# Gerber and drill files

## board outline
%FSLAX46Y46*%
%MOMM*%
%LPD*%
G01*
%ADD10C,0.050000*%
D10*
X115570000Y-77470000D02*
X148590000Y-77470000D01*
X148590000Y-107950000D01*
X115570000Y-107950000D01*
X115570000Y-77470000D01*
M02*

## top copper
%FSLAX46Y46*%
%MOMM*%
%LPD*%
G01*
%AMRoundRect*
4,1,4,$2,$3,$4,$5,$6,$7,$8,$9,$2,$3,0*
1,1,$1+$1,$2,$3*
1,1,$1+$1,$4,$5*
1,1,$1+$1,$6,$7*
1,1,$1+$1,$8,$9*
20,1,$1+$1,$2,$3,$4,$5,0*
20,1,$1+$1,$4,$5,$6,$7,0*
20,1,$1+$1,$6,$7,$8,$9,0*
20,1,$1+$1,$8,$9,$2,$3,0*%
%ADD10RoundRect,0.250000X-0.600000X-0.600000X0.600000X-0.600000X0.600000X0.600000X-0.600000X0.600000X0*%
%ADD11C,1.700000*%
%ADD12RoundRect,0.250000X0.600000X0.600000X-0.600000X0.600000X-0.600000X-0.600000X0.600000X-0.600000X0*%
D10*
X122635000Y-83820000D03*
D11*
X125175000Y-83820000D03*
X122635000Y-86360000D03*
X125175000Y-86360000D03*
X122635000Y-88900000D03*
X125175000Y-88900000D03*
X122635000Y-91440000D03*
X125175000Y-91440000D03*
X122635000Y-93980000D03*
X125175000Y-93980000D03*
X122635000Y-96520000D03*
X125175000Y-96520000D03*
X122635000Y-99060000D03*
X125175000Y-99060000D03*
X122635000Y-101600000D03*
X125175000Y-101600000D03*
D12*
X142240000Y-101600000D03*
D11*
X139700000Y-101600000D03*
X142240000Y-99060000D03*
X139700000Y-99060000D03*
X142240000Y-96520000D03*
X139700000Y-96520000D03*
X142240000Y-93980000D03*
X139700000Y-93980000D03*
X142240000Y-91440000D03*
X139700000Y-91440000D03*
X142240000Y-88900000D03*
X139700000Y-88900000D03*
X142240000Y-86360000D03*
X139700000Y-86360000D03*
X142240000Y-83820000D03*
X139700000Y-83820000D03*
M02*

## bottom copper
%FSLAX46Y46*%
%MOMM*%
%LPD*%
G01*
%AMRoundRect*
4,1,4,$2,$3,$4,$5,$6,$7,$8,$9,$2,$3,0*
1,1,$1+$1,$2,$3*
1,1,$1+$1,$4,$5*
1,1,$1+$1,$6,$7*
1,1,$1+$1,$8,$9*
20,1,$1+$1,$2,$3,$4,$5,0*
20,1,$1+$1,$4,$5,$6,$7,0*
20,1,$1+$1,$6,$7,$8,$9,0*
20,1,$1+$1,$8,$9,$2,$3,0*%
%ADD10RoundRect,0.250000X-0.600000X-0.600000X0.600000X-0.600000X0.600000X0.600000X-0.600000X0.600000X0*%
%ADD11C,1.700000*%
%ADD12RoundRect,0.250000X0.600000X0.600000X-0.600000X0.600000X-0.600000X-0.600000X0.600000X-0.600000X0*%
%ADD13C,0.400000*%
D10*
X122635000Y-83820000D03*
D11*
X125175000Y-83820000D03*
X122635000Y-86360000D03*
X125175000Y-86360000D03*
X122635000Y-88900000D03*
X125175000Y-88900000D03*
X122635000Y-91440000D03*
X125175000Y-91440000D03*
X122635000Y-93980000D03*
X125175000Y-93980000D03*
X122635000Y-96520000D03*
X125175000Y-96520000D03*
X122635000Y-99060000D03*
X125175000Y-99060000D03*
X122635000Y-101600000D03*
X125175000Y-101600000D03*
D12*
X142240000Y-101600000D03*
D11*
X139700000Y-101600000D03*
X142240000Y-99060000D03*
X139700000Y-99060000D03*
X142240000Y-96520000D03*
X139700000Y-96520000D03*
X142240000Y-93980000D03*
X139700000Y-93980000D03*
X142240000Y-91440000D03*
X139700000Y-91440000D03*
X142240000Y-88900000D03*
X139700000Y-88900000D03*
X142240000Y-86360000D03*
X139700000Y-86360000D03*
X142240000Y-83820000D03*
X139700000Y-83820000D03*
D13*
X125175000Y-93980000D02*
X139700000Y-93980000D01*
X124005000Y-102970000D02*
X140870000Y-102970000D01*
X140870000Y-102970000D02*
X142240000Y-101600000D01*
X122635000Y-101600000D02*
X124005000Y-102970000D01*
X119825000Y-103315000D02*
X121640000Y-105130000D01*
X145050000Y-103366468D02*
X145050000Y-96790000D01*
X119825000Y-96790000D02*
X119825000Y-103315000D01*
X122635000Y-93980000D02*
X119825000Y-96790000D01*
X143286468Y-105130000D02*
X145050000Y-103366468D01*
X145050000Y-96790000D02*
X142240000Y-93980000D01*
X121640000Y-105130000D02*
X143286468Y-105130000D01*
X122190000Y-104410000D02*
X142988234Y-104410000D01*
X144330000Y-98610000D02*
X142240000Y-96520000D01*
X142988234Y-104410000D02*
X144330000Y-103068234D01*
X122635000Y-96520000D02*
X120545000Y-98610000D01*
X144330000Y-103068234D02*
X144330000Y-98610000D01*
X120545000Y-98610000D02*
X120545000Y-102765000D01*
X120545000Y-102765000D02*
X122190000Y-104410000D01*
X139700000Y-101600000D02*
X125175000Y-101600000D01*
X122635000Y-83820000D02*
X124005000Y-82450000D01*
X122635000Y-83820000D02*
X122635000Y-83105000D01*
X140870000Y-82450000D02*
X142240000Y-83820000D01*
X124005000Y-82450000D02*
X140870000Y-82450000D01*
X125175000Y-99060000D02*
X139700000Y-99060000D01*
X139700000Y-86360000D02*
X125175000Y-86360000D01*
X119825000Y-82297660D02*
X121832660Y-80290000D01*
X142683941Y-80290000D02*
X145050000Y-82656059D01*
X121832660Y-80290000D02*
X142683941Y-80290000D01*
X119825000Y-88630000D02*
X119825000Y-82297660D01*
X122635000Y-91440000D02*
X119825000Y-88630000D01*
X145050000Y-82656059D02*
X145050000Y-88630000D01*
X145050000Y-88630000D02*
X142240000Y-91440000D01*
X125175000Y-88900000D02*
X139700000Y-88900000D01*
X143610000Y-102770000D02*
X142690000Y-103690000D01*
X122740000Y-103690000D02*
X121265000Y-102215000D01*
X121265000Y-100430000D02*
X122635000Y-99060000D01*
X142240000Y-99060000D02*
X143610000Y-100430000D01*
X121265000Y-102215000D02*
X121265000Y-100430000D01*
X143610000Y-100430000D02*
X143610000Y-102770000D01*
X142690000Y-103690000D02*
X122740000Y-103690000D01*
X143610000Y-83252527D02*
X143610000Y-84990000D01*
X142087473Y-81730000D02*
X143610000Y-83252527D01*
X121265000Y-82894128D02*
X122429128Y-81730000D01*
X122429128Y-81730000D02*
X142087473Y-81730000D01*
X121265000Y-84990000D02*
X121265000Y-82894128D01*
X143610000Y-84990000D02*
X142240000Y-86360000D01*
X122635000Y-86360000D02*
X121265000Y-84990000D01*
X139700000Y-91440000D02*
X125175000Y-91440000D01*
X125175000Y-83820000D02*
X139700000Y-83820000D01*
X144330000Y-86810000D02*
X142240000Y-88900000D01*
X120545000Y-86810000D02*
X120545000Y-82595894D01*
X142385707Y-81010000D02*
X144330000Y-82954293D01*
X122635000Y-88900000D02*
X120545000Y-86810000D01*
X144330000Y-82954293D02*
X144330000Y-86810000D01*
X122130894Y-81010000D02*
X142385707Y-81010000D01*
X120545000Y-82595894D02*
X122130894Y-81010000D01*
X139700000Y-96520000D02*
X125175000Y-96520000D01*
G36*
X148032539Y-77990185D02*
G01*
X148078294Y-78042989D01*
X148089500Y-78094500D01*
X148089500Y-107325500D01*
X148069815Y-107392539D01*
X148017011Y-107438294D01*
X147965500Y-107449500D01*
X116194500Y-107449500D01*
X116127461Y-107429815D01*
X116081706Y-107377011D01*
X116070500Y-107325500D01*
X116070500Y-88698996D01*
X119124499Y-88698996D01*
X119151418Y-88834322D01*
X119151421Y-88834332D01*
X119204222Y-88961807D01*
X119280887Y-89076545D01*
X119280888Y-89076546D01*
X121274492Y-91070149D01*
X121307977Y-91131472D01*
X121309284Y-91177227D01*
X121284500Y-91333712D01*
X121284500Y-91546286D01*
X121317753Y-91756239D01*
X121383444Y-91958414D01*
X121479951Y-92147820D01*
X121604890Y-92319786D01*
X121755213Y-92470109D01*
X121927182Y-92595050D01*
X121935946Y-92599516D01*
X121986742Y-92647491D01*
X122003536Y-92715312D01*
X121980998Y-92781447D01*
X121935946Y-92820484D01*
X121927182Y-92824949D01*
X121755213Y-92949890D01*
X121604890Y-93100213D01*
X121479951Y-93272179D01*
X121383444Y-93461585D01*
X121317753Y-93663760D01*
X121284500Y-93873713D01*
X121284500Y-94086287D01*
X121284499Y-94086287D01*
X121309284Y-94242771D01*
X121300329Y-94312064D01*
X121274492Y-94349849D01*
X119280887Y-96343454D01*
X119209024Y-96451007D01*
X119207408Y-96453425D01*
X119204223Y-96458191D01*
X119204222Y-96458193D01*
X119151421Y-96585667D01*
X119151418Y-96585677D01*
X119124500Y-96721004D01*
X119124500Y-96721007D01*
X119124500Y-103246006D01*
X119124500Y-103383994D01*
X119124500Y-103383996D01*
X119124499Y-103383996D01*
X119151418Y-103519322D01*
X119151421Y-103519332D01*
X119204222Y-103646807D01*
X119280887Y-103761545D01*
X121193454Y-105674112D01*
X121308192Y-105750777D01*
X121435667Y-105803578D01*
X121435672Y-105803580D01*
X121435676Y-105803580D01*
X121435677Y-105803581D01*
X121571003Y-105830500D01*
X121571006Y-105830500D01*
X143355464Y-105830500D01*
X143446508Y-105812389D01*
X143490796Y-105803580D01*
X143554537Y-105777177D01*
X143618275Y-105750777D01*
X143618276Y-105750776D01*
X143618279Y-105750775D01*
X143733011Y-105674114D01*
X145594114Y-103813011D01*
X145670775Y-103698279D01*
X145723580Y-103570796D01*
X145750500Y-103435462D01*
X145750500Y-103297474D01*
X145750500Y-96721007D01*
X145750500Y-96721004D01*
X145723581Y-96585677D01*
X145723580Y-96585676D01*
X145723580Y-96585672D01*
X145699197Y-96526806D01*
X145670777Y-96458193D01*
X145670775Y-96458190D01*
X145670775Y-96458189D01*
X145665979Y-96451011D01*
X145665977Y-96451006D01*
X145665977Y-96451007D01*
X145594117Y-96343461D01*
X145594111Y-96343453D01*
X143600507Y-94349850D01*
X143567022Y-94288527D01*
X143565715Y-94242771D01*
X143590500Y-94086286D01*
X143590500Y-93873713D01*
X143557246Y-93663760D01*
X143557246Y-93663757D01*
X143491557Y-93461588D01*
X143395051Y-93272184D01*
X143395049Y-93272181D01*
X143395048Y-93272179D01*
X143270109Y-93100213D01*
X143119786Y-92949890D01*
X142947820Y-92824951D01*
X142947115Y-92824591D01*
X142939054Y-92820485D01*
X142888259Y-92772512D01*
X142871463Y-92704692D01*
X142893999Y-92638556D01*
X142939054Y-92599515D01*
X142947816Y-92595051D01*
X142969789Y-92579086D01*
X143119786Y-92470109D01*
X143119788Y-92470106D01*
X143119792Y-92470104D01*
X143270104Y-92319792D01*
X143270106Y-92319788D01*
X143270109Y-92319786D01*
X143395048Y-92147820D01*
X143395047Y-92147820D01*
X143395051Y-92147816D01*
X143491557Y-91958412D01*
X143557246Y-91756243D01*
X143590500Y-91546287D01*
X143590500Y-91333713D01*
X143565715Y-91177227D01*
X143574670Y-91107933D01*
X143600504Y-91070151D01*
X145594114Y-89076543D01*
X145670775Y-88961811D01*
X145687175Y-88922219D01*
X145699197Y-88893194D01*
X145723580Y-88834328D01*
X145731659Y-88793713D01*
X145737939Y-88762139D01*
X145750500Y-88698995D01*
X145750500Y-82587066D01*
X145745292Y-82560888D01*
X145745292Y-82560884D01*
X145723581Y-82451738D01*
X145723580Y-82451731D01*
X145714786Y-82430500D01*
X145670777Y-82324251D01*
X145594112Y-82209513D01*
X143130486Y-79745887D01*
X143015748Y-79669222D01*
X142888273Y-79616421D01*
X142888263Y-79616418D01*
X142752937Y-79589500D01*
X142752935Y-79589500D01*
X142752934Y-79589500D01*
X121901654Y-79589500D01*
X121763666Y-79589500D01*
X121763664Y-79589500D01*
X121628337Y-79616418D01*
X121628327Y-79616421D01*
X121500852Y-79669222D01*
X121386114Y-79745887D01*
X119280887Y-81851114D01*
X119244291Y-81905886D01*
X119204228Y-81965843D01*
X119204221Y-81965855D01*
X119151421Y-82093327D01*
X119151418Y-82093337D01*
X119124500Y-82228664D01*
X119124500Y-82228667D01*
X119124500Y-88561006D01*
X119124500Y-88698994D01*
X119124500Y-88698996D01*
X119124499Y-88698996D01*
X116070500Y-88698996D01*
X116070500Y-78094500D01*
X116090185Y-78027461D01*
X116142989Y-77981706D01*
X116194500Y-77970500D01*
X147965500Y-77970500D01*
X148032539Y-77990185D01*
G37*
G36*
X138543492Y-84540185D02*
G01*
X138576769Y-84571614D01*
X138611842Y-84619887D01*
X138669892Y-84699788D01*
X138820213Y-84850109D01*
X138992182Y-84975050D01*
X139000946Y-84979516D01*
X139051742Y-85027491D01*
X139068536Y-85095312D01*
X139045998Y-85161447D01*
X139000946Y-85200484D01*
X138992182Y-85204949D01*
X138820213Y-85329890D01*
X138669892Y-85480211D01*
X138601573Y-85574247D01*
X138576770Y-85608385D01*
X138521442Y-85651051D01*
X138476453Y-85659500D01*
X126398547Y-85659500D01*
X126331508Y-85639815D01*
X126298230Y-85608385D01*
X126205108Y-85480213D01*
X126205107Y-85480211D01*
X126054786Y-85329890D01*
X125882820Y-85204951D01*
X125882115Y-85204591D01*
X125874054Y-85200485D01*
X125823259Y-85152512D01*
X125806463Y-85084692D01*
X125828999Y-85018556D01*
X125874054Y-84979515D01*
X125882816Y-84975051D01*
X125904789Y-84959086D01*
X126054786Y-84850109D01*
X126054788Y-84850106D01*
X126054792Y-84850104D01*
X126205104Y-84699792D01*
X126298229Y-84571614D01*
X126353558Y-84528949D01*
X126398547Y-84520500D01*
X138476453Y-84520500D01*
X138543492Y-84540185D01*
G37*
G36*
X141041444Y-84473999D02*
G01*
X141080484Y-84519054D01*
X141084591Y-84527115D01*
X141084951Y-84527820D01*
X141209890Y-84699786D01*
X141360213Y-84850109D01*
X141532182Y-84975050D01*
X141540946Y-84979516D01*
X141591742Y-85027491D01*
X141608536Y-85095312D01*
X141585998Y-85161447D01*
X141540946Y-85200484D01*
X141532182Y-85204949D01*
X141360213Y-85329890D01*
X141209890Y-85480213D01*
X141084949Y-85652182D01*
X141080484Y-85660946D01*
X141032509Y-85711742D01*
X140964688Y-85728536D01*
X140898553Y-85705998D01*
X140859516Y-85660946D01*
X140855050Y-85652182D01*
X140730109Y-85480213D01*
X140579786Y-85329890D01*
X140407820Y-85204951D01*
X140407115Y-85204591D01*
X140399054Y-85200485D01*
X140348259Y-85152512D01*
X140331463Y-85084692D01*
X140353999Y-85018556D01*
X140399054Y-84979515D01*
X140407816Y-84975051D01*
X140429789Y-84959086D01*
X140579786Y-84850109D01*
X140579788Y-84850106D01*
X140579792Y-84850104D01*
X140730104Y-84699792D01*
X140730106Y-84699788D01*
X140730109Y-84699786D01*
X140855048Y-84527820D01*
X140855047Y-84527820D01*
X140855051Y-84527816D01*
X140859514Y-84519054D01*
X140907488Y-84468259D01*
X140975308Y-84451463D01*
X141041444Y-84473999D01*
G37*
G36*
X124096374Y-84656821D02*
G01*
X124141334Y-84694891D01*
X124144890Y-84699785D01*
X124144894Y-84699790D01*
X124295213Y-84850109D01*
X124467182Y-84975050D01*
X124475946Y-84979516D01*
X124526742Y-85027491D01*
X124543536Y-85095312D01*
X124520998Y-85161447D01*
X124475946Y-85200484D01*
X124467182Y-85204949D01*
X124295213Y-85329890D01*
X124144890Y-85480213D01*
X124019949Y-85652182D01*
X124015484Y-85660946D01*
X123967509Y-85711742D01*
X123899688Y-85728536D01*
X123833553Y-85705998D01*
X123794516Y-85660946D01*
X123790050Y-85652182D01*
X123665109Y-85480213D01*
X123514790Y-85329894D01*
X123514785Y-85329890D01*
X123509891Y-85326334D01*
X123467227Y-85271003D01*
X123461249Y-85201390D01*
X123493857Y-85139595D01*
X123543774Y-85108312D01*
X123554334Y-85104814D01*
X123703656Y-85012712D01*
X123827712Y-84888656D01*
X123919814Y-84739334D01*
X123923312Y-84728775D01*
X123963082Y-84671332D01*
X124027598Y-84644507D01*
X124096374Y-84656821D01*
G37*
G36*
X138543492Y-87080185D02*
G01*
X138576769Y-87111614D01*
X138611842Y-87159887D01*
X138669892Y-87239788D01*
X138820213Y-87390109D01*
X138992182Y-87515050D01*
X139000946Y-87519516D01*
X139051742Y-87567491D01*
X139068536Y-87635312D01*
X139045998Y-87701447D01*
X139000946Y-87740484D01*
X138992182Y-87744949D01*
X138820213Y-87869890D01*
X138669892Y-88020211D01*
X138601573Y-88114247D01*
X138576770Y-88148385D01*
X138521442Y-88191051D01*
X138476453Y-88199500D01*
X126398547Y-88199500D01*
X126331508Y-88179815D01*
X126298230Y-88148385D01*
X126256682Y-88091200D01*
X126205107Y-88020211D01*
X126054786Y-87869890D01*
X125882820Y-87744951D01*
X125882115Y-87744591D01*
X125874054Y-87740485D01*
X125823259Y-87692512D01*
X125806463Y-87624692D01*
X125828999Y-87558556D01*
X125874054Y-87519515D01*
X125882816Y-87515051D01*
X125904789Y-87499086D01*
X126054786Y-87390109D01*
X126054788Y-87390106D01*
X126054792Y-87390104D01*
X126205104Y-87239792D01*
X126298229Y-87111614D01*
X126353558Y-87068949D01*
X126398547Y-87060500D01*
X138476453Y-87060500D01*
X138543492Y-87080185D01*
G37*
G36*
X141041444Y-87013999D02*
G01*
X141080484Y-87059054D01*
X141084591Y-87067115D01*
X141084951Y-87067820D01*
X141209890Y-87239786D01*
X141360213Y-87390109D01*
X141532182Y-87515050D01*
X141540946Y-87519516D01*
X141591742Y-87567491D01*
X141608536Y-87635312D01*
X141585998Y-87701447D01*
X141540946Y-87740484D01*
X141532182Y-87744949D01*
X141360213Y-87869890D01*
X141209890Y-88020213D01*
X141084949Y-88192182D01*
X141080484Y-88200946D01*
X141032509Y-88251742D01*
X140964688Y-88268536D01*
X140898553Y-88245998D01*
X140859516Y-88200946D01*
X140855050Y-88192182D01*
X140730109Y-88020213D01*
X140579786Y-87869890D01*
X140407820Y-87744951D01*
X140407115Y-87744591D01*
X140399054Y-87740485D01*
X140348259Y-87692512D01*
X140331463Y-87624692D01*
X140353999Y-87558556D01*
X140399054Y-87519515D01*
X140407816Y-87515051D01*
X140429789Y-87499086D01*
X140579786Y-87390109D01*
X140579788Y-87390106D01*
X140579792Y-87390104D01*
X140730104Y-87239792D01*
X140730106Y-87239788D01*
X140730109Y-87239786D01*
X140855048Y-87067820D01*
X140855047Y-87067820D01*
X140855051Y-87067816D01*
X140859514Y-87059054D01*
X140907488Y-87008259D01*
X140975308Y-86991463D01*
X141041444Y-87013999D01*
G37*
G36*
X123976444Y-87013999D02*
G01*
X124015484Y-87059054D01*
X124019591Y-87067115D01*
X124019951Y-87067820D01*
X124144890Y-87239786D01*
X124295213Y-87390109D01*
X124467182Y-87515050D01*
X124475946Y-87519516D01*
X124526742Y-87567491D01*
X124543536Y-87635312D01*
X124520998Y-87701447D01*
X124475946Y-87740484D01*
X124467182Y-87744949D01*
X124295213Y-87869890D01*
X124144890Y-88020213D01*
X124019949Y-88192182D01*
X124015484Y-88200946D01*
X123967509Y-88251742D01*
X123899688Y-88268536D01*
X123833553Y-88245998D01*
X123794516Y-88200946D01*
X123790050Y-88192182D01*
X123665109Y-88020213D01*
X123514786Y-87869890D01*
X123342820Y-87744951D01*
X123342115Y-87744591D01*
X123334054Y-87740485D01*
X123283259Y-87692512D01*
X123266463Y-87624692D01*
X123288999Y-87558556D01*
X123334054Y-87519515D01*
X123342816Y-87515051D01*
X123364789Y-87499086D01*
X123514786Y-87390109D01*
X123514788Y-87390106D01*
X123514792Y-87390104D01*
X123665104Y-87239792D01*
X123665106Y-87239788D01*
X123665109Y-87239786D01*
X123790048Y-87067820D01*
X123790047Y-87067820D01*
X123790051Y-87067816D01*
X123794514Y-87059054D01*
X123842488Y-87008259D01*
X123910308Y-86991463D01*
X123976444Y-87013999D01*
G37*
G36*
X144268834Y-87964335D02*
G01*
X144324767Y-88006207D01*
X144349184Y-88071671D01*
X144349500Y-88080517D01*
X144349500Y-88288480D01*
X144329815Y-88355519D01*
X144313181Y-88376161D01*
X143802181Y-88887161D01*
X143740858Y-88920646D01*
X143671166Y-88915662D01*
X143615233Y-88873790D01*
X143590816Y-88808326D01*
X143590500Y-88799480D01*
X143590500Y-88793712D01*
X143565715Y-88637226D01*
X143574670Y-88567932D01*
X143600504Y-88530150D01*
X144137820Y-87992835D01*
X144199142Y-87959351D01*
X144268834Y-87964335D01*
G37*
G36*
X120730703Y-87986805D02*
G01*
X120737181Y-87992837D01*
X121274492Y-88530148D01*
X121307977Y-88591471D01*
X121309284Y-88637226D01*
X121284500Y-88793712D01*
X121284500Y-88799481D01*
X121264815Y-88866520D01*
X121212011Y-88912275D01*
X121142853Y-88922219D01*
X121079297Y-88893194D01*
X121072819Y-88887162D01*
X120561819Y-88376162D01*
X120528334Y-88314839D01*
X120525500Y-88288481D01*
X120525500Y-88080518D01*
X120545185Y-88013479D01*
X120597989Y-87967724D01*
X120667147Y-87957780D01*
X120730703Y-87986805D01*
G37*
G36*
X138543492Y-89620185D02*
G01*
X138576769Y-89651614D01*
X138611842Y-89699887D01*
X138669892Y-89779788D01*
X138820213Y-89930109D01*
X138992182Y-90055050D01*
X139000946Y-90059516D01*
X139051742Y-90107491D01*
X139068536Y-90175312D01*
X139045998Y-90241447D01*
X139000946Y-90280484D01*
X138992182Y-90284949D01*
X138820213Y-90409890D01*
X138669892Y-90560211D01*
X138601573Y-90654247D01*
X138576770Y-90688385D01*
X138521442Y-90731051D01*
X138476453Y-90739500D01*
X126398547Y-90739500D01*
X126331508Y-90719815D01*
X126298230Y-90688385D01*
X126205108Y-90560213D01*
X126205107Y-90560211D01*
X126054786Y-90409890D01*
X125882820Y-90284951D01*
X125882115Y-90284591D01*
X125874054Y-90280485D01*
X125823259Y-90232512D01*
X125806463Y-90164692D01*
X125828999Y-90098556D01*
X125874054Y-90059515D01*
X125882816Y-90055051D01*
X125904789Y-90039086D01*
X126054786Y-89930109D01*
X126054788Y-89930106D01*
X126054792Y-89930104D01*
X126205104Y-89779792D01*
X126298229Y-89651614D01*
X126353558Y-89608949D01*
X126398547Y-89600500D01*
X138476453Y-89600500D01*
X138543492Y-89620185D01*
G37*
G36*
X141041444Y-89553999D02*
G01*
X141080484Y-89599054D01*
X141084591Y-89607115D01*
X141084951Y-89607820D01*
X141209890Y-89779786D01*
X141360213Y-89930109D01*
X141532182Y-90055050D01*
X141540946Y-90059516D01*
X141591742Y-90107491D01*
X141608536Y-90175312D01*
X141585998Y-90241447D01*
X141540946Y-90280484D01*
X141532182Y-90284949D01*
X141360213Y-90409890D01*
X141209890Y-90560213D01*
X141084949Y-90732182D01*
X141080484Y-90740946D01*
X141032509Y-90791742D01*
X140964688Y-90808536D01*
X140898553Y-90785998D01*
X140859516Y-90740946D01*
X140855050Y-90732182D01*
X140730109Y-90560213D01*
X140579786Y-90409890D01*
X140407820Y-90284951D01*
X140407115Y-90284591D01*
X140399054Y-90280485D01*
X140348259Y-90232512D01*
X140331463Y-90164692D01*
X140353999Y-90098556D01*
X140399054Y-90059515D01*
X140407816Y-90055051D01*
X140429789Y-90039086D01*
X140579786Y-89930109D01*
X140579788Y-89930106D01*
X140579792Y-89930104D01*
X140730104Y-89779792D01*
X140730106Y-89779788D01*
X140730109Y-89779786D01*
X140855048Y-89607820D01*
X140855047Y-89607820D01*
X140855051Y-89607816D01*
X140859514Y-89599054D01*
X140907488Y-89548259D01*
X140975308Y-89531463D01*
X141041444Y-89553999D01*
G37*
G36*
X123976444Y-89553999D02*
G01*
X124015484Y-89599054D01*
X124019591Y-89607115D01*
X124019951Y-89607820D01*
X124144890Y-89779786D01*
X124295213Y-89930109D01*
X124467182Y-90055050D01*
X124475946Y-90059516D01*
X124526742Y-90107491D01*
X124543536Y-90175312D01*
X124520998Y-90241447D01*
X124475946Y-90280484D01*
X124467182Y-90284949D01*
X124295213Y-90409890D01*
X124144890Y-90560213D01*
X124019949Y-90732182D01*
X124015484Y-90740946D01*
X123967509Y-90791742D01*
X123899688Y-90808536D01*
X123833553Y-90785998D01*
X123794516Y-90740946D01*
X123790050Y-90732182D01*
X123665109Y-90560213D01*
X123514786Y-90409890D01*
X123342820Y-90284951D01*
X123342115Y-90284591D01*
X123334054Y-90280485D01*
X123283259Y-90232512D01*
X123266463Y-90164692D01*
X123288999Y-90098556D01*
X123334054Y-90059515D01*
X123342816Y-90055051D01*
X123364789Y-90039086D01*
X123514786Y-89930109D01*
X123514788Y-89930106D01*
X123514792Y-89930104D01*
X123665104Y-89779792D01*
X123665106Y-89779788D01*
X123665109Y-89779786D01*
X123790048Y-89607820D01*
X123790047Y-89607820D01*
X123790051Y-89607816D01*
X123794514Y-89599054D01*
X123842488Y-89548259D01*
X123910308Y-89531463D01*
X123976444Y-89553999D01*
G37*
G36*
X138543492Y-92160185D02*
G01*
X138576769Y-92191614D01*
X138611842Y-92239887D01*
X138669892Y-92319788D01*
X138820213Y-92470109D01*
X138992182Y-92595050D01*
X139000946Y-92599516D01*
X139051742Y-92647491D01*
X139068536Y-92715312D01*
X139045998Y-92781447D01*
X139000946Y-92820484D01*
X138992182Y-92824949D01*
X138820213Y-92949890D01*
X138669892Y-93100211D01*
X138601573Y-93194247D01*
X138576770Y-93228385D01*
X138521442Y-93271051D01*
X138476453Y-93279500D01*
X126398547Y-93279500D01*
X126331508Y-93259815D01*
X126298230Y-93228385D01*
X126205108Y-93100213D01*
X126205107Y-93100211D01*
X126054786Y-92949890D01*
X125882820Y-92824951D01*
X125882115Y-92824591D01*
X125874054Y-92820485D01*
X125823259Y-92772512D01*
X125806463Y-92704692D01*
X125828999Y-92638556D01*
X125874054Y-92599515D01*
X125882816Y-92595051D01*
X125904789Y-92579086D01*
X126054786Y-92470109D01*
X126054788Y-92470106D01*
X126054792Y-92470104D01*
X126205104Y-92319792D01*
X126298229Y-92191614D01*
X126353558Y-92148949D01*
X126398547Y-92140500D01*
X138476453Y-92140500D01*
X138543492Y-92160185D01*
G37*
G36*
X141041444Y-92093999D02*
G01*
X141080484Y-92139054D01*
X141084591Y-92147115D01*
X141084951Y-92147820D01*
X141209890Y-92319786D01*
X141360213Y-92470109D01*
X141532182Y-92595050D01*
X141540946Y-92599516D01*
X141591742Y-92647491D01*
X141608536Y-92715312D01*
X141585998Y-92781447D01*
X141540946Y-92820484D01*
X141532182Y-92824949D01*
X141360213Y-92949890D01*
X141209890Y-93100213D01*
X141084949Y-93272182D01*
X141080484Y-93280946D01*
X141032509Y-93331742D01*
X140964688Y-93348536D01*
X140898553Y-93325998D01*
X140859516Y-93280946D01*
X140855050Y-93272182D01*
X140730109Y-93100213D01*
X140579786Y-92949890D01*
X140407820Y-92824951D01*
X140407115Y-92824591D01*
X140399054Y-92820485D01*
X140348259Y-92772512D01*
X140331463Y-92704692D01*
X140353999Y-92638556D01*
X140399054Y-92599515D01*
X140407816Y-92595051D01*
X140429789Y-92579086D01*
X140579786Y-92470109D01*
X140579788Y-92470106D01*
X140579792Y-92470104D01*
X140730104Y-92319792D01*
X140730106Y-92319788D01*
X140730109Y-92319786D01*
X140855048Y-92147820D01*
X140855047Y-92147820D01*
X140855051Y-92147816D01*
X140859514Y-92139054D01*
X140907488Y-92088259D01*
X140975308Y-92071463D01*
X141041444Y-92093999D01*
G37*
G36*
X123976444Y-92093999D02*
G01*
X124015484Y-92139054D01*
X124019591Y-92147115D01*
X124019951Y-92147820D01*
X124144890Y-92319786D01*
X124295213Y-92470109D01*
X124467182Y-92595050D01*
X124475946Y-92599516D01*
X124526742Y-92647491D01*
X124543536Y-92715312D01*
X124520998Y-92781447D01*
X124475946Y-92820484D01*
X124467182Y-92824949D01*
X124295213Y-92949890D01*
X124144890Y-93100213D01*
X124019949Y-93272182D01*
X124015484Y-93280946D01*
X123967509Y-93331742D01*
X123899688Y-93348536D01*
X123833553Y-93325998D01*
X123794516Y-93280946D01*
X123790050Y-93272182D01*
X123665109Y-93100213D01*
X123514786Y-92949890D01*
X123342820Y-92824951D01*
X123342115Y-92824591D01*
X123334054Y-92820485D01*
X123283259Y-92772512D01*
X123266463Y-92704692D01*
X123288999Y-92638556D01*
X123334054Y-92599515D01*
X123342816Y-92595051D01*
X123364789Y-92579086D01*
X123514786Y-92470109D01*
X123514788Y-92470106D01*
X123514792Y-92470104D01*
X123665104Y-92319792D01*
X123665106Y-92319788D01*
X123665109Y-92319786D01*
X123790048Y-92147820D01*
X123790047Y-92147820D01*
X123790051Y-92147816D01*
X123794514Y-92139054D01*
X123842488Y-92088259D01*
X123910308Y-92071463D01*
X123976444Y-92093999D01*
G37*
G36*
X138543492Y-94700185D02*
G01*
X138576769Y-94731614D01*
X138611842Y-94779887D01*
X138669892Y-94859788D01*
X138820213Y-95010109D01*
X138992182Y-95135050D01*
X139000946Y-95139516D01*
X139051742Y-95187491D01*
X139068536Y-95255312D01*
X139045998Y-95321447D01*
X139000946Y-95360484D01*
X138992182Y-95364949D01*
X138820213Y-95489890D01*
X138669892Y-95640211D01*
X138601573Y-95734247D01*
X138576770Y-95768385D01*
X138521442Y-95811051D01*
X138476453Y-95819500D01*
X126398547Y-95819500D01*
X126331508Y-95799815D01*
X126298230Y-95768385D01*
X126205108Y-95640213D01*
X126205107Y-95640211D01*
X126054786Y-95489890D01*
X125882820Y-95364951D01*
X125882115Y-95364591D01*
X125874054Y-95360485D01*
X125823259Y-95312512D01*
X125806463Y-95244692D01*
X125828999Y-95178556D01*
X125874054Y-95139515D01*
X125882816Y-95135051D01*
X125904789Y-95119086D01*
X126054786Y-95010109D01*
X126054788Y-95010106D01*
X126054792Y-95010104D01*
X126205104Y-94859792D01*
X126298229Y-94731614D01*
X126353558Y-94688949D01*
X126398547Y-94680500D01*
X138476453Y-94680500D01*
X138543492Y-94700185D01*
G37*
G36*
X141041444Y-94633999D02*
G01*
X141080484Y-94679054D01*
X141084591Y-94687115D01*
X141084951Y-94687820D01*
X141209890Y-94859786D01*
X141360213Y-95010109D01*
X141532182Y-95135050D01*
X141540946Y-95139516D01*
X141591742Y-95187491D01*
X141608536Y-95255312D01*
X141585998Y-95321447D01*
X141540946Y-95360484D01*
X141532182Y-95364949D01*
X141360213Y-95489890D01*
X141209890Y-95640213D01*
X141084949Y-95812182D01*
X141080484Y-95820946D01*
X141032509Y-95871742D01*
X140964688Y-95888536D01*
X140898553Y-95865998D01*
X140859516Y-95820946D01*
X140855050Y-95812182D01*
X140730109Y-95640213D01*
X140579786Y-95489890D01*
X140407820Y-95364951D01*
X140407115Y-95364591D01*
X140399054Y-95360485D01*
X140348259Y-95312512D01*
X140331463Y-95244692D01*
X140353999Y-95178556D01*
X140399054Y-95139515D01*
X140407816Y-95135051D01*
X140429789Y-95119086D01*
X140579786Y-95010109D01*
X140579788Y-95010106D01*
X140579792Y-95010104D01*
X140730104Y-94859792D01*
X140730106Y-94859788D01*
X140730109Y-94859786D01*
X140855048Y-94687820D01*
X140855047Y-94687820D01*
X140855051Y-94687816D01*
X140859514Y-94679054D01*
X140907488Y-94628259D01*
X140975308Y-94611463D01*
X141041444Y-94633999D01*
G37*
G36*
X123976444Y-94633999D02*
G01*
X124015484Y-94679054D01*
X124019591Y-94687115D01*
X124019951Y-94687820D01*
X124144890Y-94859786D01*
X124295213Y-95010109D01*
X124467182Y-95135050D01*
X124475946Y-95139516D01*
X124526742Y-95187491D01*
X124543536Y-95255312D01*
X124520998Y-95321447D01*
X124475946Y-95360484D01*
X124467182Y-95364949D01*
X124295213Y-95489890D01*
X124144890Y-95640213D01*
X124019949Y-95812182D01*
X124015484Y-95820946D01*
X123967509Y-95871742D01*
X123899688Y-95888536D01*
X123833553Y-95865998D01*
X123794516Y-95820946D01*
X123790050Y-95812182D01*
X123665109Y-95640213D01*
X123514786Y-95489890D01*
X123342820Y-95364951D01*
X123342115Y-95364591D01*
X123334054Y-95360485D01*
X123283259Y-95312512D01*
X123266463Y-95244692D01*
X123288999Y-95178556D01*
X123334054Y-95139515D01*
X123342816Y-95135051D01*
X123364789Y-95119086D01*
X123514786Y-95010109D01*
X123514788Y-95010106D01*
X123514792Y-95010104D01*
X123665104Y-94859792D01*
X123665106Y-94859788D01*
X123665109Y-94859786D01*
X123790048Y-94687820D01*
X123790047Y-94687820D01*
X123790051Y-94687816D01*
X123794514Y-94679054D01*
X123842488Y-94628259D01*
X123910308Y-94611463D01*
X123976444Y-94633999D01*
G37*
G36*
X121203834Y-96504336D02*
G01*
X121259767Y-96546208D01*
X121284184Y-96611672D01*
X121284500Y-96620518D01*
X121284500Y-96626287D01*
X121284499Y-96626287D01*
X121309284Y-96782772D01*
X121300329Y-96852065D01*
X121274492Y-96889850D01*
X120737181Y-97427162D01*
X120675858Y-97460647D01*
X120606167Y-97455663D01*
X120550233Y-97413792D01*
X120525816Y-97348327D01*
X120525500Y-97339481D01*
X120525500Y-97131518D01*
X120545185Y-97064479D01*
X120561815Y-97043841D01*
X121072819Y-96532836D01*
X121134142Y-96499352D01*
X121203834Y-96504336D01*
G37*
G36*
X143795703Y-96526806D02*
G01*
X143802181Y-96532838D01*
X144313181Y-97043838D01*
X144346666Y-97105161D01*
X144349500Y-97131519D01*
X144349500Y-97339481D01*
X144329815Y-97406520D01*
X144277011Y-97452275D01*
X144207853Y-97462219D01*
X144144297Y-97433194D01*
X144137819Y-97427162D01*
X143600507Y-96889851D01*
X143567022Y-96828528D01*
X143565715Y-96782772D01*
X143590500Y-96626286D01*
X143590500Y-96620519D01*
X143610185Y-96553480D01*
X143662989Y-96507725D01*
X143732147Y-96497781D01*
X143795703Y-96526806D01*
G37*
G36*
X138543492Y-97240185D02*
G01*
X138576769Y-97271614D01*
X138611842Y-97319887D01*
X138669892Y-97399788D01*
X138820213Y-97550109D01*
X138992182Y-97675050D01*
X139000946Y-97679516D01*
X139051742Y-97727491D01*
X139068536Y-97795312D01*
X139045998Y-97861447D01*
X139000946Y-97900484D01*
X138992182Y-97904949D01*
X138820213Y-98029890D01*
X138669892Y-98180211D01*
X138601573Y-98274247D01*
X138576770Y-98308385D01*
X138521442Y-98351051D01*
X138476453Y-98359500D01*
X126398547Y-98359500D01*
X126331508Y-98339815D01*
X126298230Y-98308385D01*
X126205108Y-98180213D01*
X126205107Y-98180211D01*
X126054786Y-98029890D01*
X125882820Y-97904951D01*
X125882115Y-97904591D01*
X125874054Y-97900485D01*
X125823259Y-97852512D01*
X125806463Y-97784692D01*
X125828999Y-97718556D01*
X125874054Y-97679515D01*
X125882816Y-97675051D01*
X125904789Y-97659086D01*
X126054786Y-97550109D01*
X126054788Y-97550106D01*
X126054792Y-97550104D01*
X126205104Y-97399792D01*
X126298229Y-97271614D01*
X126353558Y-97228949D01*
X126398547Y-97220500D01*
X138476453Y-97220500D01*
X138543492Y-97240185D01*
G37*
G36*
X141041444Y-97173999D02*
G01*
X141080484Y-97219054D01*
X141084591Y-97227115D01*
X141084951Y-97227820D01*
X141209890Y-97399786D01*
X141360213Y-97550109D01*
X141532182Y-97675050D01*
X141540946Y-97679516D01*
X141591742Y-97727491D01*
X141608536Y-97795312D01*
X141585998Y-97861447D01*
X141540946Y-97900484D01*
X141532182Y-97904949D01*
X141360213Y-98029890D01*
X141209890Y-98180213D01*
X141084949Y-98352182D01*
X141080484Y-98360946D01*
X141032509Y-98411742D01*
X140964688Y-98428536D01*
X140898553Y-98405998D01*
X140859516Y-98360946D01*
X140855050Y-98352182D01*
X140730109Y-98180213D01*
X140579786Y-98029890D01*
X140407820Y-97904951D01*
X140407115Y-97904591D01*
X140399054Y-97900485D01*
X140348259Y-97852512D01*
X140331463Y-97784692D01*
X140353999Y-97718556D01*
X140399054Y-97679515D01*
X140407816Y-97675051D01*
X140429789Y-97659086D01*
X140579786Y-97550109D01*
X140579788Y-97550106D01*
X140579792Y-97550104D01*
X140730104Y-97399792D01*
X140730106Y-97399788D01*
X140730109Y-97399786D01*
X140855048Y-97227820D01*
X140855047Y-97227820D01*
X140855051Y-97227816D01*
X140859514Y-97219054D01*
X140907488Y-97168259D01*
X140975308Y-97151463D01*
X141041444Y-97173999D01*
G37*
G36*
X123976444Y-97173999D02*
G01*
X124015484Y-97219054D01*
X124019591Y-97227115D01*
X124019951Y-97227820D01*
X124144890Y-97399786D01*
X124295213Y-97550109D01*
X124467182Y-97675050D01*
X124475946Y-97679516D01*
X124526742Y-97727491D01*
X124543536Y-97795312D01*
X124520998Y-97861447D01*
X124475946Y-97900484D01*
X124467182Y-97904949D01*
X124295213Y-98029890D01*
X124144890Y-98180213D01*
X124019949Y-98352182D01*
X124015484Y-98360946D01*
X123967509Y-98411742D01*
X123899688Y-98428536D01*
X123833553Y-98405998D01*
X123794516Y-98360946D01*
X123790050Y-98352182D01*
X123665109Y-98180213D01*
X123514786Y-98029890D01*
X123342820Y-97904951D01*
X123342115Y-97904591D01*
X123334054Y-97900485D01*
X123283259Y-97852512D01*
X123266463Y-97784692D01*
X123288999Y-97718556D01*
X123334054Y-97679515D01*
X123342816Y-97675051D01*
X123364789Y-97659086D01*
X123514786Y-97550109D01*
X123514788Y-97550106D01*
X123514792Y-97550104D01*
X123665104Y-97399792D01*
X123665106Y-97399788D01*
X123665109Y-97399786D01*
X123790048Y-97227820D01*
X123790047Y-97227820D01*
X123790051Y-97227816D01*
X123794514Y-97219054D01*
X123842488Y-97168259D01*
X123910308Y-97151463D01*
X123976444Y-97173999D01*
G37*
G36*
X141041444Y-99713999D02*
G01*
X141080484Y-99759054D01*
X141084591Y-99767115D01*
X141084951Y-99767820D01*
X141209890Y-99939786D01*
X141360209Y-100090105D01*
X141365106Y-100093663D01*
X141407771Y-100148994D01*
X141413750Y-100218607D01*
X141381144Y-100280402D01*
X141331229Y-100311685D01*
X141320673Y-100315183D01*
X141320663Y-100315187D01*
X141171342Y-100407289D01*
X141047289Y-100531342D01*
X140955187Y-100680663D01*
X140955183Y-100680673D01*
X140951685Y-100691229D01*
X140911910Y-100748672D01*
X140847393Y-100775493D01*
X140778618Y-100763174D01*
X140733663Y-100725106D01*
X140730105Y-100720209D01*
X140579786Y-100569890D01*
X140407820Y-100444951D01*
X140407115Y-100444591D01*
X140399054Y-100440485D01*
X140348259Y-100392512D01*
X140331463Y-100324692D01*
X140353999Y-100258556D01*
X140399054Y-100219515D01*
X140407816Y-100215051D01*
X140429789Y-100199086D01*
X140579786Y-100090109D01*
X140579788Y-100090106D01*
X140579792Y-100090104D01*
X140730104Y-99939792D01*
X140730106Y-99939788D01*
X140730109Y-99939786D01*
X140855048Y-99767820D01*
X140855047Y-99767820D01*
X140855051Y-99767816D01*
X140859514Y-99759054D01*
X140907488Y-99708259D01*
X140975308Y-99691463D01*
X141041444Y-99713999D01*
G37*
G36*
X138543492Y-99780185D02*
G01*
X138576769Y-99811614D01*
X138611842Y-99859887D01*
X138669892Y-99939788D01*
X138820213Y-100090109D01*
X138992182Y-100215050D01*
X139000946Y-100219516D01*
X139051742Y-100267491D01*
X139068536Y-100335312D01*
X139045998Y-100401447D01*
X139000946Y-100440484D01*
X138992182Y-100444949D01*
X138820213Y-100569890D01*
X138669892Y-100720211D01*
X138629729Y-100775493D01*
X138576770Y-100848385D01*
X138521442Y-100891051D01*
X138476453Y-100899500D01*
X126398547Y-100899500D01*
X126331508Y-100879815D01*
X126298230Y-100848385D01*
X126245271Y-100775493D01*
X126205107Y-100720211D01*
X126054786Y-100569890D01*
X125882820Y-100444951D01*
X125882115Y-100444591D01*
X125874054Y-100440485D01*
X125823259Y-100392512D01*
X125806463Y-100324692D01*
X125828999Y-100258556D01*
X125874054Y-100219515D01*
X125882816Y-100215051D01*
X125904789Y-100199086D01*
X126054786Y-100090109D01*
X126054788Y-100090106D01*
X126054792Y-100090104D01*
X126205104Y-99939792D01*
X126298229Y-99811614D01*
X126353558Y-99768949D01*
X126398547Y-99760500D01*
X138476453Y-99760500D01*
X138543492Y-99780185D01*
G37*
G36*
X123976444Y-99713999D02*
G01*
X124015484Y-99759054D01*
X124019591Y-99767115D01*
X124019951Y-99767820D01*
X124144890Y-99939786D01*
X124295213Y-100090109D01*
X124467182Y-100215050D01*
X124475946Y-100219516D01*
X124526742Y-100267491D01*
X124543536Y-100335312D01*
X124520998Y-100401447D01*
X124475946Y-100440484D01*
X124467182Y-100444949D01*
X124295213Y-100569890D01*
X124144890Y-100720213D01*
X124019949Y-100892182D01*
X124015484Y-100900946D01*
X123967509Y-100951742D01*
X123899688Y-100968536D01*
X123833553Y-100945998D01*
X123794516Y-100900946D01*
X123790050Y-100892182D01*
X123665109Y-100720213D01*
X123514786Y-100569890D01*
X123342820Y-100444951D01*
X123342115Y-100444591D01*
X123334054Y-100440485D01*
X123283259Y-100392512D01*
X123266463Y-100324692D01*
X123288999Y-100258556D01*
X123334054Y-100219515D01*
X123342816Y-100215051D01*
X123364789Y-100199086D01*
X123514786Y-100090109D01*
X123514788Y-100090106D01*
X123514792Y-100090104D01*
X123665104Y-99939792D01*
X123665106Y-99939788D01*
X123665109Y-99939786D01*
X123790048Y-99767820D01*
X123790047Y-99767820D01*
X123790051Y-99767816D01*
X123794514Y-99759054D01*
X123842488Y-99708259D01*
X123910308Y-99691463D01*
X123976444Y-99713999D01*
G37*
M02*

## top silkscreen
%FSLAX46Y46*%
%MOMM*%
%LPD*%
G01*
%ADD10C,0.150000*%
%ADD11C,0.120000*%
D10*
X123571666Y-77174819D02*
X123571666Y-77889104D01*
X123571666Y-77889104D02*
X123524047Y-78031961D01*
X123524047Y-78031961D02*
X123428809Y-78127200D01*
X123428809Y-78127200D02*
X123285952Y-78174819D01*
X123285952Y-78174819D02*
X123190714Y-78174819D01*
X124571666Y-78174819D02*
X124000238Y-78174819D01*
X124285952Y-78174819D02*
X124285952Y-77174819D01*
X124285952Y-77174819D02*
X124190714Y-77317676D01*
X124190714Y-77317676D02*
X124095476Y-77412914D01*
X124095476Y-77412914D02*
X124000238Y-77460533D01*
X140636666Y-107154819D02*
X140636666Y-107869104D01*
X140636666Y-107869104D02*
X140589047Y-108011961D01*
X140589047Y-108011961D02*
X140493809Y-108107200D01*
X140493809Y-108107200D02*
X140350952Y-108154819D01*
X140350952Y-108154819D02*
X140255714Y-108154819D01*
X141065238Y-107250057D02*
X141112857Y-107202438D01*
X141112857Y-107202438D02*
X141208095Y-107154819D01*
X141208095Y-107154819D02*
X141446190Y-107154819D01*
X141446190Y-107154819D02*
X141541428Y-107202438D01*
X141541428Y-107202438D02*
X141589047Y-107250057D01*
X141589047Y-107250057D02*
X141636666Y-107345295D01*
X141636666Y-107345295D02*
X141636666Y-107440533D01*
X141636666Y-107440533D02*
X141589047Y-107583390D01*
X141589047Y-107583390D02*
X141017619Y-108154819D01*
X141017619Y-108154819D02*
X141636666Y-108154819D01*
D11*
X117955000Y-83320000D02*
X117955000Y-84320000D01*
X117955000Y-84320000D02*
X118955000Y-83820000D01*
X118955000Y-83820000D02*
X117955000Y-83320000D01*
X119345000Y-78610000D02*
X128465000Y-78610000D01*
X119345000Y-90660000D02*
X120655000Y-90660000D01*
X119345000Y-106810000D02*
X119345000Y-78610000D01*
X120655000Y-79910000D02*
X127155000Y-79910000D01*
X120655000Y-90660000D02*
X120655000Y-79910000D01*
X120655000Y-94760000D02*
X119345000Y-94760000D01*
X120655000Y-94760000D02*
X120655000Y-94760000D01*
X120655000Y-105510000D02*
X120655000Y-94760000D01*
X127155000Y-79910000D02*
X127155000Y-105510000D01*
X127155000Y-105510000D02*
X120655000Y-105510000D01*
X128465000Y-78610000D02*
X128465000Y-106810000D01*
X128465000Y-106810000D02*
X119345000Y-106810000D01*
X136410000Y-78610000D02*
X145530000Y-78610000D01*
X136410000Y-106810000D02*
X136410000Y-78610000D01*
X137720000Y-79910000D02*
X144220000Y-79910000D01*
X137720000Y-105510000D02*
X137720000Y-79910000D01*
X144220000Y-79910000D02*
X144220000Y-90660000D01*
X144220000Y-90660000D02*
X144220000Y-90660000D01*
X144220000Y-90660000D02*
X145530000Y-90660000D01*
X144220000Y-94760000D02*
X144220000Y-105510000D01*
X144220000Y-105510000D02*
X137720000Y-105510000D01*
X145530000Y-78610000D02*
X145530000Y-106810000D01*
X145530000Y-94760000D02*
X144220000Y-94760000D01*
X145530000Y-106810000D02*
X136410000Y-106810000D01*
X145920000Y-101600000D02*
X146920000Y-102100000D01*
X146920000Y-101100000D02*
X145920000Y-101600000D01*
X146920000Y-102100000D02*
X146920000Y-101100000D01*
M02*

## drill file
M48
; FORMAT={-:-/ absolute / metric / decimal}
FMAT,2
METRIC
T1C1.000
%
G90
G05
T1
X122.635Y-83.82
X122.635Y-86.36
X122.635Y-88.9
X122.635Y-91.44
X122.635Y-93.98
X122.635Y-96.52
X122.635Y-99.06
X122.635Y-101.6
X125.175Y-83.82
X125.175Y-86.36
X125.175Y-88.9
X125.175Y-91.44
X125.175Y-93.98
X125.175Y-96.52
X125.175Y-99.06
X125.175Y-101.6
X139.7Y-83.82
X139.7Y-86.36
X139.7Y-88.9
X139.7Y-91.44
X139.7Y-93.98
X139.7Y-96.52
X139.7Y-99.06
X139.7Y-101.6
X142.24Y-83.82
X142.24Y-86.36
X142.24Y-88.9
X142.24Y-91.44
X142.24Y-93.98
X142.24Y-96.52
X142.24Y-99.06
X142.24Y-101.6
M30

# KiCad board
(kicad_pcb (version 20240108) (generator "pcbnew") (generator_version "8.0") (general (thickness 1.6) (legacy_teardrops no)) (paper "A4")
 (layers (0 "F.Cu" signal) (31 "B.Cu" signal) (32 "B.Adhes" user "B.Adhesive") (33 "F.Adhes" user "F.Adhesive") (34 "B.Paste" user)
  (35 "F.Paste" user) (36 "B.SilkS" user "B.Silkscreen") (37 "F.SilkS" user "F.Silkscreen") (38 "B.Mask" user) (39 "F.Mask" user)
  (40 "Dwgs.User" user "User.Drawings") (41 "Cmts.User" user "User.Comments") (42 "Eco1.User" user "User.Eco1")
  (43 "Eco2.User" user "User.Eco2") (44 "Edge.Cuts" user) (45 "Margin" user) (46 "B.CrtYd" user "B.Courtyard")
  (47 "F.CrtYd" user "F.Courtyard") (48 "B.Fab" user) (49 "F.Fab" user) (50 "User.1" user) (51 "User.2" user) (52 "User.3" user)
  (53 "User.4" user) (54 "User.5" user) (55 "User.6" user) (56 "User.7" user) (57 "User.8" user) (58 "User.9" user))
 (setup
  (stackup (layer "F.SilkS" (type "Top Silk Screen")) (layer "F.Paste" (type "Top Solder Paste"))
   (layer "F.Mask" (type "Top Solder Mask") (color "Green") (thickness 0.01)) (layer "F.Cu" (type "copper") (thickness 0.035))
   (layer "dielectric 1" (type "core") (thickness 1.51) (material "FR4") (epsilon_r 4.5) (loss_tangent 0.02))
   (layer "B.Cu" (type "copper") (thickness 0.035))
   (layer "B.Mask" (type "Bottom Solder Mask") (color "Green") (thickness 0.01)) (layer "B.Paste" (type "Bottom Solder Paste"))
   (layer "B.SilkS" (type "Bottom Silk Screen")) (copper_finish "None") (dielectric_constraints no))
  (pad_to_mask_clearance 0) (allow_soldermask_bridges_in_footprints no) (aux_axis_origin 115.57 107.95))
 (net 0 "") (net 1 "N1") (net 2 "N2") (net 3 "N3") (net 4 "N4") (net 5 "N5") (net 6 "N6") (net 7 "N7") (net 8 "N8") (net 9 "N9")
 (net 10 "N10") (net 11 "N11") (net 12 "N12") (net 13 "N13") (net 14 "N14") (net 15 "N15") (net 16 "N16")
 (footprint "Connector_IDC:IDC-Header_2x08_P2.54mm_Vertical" (layer "F.Cu") (at 122.635 83.82)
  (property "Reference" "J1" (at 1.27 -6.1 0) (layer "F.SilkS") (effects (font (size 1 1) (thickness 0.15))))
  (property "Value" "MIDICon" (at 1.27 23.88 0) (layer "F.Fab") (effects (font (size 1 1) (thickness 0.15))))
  (fp_line (start -4.68 -0.5) (end -4.68 0.5) (stroke (width 0.12) (type solid)) (layer "F.SilkS"))
  (fp_line (start -4.68 0.5) (end -3.68 0) (stroke (width 0.12) (type solid)) (layer "F.SilkS"))
  (fp_line (start -3.68 0) (end -4.68 -0.5) (stroke (width 0.12) (type solid)) (layer "F.SilkS"))
  (fp_line (start -3.29 -5.21) (end 5.83 -5.21) (stroke (width 0.12) (type solid)) (layer "F.SilkS"))
  (fp_line (start -3.29 6.84) (end -1.98 6.84) (stroke (width 0.12) (type solid)) (layer "F.SilkS"))
  (fp_line (start -3.29 22.99) (end -3.29 -5.21) (stroke (width 0.12) (type solid)) (layer "F.SilkS"))
  (fp_line (start -1.98 -3.91) (end 4.52 -3.91) (stroke (width 0.12) (type solid)) (layer "F.SilkS"))
  (fp_line (start -1.98 6.84) (end -1.98 -3.91) (stroke (width 0.12) (type solid)) (layer "F.SilkS"))
  (fp_line (start -1.98 10.94) (end -3.29 10.94) (stroke (width 0.12) (type solid)) (layer "F.SilkS"))
  (fp_line (start -1.98 10.94) (end -1.98 10.94) (stroke (width 0.12) (type solid)) (layer "F.SilkS"))
  (fp_line (start -1.98 21.69) (end -1.98 10.94) (stroke (width 0.12) (type solid)) (layer "F.SilkS"))
  (fp_line (start 4.52 -3.91) (end 4.52 21.69) (stroke (width 0.12) (type solid)) (layer "F.SilkS"))
  (fp_line (start 4.52 21.69) (end -1.98 21.69) (stroke (width 0.12) (type solid)) (layer "F.SilkS"))
  (fp_line (start 5.83 -5.21) (end 5.83 22.99) (stroke (width 0.12) (type solid)) (layer "F.SilkS"))
  (fp_line (start 5.83 22.99) (end -3.29 22.99) (stroke (width 0.12) (type solid)) (layer "F.SilkS"))
  (pad "1" thru_hole roundrect (at 0 0) (size 1.7 1.7) (drill 1) (layers "*.Cu" "*.Mask") (remove_unused_layers no)
   (roundrect_rratio 0.147059) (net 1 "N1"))
  (pad "2" thru_hole circle (at 2.54 0) (size 1.7 1.7) (drill 1) (layers "*.Cu" "*.Mask") (remove_unused_layers no) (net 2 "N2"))
  (pad "3" thru_hole circle (at 0 2.54) (size 1.7 1.7) (drill 1) (layers "*.Cu" "*.Mask") (remove_unused_layers no) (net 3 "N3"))
  (pad "4" thru_hole circle (at 2.54 2.54) (size 1.7 1.7) (drill 1) (layers "*.Cu" "*.Mask") (remove_unused_layers no) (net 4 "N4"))
  (pad "5" thru_hole circle (at 0 5.08) (size 1.7 1.7) (drill 1) (layers "*.Cu" "*.Mask") (remove_unused_layers no) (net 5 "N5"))
  (pad "6" thru_hole circle (at 2.54 5.08) (size 1.7 1.7) (drill 1) (layers "*.Cu" "*.Mask") (remove_unused_layers no) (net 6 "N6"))
  (pad "7" thru_hole circle (at 0 7.62) (size 1.7 1.7) (drill 1) (layers "*.Cu" "*.Mask") (remove_unused_layers no) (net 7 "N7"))
  (pad "8" thru_hole circle (at 2.54 7.62) (size 1.7 1.7) (drill 1) (layers "*.Cu" "*.Mask") (remove_unused_layers no) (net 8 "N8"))
  (pad "9" thru_hole circle (at 0 10.16) (size 1.7 1.7) (drill 1) (layers "*.Cu" "*.Mask") (remove_unused_layers no) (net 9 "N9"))
  (pad "10" thru_hole circle (at 2.54 10.16) (size 1.7 1.7) (drill 1) (layers "*.Cu" "*.Mask") (remove_unused_layers no) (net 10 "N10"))
  (pad "11" thru_hole circle (at 0 12.7) (size 1.7 1.7) (drill 1) (layers "*.Cu" "*.Mask") (remove_unused_layers no) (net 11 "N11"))
  (pad "12" thru_hole circle (at 2.54 12.7) (size 1.7 1.7) (drill 1) (layers "*.Cu" "*.Mask") (remove_unused_layers no) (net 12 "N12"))
  (pad "13" thru_hole circle (at 0 15.24) (size 1.7 1.7) (drill 1) (layers "*.Cu" "*.Mask") (remove_unused_layers no) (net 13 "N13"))
  (pad "14" thru_hole circle (at 2.54 15.24) (size 1.7 1.7) (drill 1) (layers "*.Cu" "*.Mask") (remove_unused_layers no) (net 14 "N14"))
  (pad "15" thru_hole circle (at 0 17.78) (size 1.7 1.7) (drill 1) (layers "*.Cu" "*.Mask") (remove_unused_layers no) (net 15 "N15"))
  (pad "16" thru_hole circle (at 2.54 17.78) (size 1.7 1.7) (drill 1) (layers "*.Cu" "*.Mask") (remove_unused_layers no) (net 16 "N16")))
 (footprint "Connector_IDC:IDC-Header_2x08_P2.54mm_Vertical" (layer "F.Cu") (at 142.24 101.6 180)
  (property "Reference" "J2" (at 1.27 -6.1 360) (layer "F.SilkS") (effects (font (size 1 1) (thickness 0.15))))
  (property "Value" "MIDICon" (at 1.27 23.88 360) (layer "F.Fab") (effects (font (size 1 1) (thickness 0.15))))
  (fp_line (start 5.83 22.99) (end -3.29 22.99) (stroke (width 0.12) (type solid)) (layer "F.SilkS"))
  (fp_line (start 5.83 -5.21) (end 5.83 22.99) (stroke (width 0.12) (type solid)) (layer "F.SilkS"))
  (fp_line (start 4.52 21.69) (end -1.98 21.69) (stroke (width 0.12) (type solid)) (layer "F.SilkS"))
  (fp_line (start 4.52 -3.91) (end 4.52 21.69) (stroke (width 0.12) (type solid)) (layer "F.SilkS"))
  (fp_line (start -1.98 21.69) (end -1.98 10.94) (stroke (width 0.12) (type solid)) (layer "F.SilkS"))
  (fp_line (start -1.98 10.94) (end -1.98 10.94) (stroke (width 0.12) (type solid)) (layer "F.SilkS"))
  (fp_line (start -1.98 10.94) (end -3.29 10.94) (stroke (width 0.12) (type solid)) (layer "F.SilkS"))
  (fp_line (start -1.98 6.84) (end -1.98 -3.91) (stroke (width 0.12) (type solid)) (layer "F.SilkS"))
  (fp_line (start -1.98 -3.91) (end 4.52 -3.91) (stroke (width 0.12) (type solid)) (layer "F.SilkS"))
  (fp_line (start -3.29 22.99) (end -3.29 -5.21) (stroke (width 0.12) (type solid)) (layer "F.SilkS"))
  (fp_line (start -3.29 6.84) (end -1.98 6.84) (stroke (width 0.12) (type solid)) (layer "F.SilkS"))
  (fp_line (start -3.29 -5.21) (end 5.83 -5.21) (stroke (width 0.12) (type solid)) (layer "F.SilkS"))
  (fp_line (start -3.68 0) (end -4.68 -0.5) (stroke (width 0.12) (type solid)) (layer "F.SilkS"))
  (fp_line (start -4.68 0.5) (end -3.68 0) (stroke (width 0.12) (type solid)) (layer "F.SilkS"))
  (fp_line (start -4.68 -0.5) (end -4.68 0.5) (stroke (width 0.12) (type solid)) (layer "F.SilkS"))
  (pad "1" thru_hole roundrect (at 0 0 180) (size 1.7 1.7) (drill 1) (layers "*.Cu" "*.Mask") (remove_unused_layers no)
   (roundrect_rratio 0.147059) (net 15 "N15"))
  (pad "2" thru_hole circle (at 2.54 0 180) (size 1.7 1.7) (drill 1) (layers "*.Cu" "*.Mask") (remove_unused_layers no) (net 16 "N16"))
  (pad "3" thru_hole circle (at 0 2.54 180) (size 1.7 1.7) (drill 1) (layers "*.Cu" "*.Mask") (remove_unused_layers no) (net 13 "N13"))
  (pad "4" thru_hole circle (at 2.54 2.54 180) (size 1.7 1.7) (drill 1) (layers "*.Cu" "*.Mask") (remove_unused_layers no) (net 14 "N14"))
  (pad "5" thru_hole circle (at 0 5.08 180) (size 1.7 1.7) (drill 1) (layers "*.Cu" "*.Mask") (remove_unused_layers no) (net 11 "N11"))
  (pad "6" thru_hole circle (at 2.54 5.08 180) (size 1.7 1.7) (drill 1) (layers "*.Cu" "*.Mask") (remove_unused_layers no) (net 12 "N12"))
  (pad "7" thru_hole circle (at 0 7.62 180) (size 1.7 1.7) (drill 1) (layers "*.Cu" "*.Mask") (remove_unused_layers no) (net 9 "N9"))
  (pad "8" thru_hole circle (at 2.54 7.62 180) (size 1.7 1.7) (drill 1) (layers "*.Cu" "*.Mask") (remove_unused_layers no) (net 10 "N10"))
  (pad "9" thru_hole circle (at 0 10.16 180) (size 1.7 1.7) (drill 1) (layers "*.Cu" "*.Mask") (remove_unused_layers no) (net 7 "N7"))
  (pad "10" thru_hole circle (at 2.54 10.16 180) (size 1.7 1.7) (drill 1) (layers "*.Cu" "*.Mask") (remove_unused_layers no) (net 8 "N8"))
  (pad "11" thru_hole circle (at 0 12.7 180) (size 1.7 1.7) (drill 1) (layers "*.Cu" "*.Mask") (remove_unused_layers no) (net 5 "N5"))
  (pad "12" thru_hole circle (at 2.54 12.7 180) (size 1.7 1.7) (drill 1) (layers "*.Cu" "*.Mask") (remove_unused_layers no) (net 6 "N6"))
  (pad "13" thru_hole circle (at 0 15.24 180) (size 1.7 1.7) (drill 1) (layers "*.Cu" "*.Mask") (remove_unused_layers no) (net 3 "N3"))
  (pad "14" thru_hole circle (at 2.54 15.24 180) (size 1.7 1.7) (drill 1) (layers "*.Cu" "*.Mask") (remove_unused_layers no) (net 4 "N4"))
  (pad "15" thru_hole circle (at 0 17.78 180) (size 1.7 1.7) (drill 1) (layers "*.Cu" "*.Mask") (remove_unused_layers no) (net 1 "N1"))
  (pad "16" thru_hole circle (at 2.54 17.78 180) (size 1.7 1.7) (drill 1) (layers "*.Cu" "*.Mask") (remove_unused_layers no) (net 2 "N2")))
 (gr_rect (start 115.57 77.47) (end 148.59 107.95) (stroke (width 0.05) (type default)) (fill none) (layer "Edge.Cuts"))
 (segment (start 125.175 93.98) (end 139.7 93.98) (width 0.4) (layer "B.Cu") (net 10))
 (segment (start 124.005 102.97) (end 140.87 102.97) (width 0.4) (layer "B.Cu") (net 15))
 (segment (start 140.87 102.97) (end 142.24 101.6) (width 0.4) (layer "B.Cu") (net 15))
 (segment (start 122.635 101.6) (end 124.005 102.97) (width 0.4) (layer "B.Cu") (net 15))
 (segment (start 119.825 103.315) (end 121.64 105.13) (width 0.4) (layer "B.Cu") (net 9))
 (segment (start 145.05 103.366468) (end 145.05 96.79) (width 0.4) (layer "B.Cu") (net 9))
 (segment (start 119.825 96.79) (end 119.825 103.315) (width 0.4) (layer "B.Cu") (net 9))
 (segment (start 122.635 93.98) (end 119.825 96.79) (width 0.4) (layer "B.Cu") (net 9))
 (segment (start 143.286468 105.13) (end 145.05 103.366468) (width 0.4) (layer "B.Cu") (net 9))
 (segment (start 145.05 96.79) (end 142.24 93.98) (width 0.4) (layer "B.Cu") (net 9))
 (segment (start 121.64 105.13) (end 143.286468 105.13) (width 0.4) (layer "B.Cu") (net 9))
 (segment (start 122.19 104.41) (end 142.988234 104.41) (width 0.4) (layer "B.Cu") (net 11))
 (segment (start 144.33 98.61) (end 142.24 96.52) (width 0.4) (layer "B.Cu") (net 11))
 (segment (start 142.988234 104.41) (end 144.33 103.068234) (width 0.4) (layer "B.Cu") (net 11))
 (segment (start 122.635 96.52) (end 120.545 98.61) (width 0.4) (layer "B.Cu") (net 11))
 (segment (start 144.33 103.068234) (end 144.33 98.61) (width 0.4) (layer "B.Cu") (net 11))
 (segment (start 120.545 98.61) (end 120.545 102.765) (width 0.4) (layer "B.Cu") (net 11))
 (segment (start 120.545 102.765) (end 122.19 104.41) (width 0.4) (layer "B.Cu") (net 11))
 (segment (start 139.7 101.6) (end 125.175 101.6) (width 0.4) (layer "B.Cu") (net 16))
 (segment (start 122.635 83.82) (end 124.005 82.45) (width 0.4) (layer "B.Cu") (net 1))
 (segment (start 122.635 83.82) (end 122.635 83.105) (width 0.4) (layer "B.Cu") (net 1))
 (segment (start 140.87 82.45) (end 142.24 83.82) (width 0.4) (layer "B.Cu") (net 1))
 (segment (start 124.005 82.45) (end 140.87 82.45) (width 0.4) (layer "B.Cu") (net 1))
 (segment (start 125.175 99.06) (end 139.7 99.06) (width 0.4) (layer "B.Cu") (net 14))
 (segment (start 139.7 86.36) (end 125.175 86.36) (width 0.4) (layer "B.Cu") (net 4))
 (segment (start 119.825 82.29766) (end 121.83266 80.29) (width 0.4) (layer "B.Cu") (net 7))
 (segment (start 142.683941 80.29) (end 145.05 82.656059) (width 0.4) (layer "B.Cu") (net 7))
 (segment (start 121.83266 80.29) (end 142.683941 80.29) (width 0.4) (layer "B.Cu") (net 7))
 (segment (start 119.825 88.63) (end 119.825 82.29766) (width 0.4) (layer "B.Cu") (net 7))
 (segment (start 122.635 91.44) (end 119.825 88.63) (width 0.4) (layer "B.Cu") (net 7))
 (segment (start 145.05 82.656059) (end 145.05 88.63) (width 0.4) (layer "B.Cu") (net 7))
 (segment (start 145.05 88.63) (end 142.24 91.44) (width 0.4) (layer "B.Cu") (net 7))
 (segment (start 125.175 88.9) (end 139.7 88.9) (width 0.4) (layer "B.Cu") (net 6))
 (segment (start 143.61 102.77) (end 142.69 103.69) (width 0.4) (layer "B.Cu") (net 13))
 (segment (start 122.74 103.69) (end 121.265 102.215) (width 0.4) (layer "B.Cu") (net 13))
 (segment (start 121.265 100.43) (end 122.635 99.06) (width 0.4) (layer "B.Cu") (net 13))
 (segment (start 142.24 99.06) (end 143.61 100.43) (width 0.4) (layer "B.Cu") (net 13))
 (segment (start 121.265 102.215) (end 121.265 100.43) (width 0.4) (layer "B.Cu") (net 13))
 (segment (start 143.61 100.43) (end 143.61 102.77) (width 0.4) (layer "B.Cu") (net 13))
 (segment (start 142.69 103.69) (end 122.74 103.69) (width 0.4) (layer "B.Cu") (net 13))
 (segment (start 143.61 83.252527) (end 143.61 84.99) (width 0.4) (layer "B.Cu") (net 3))
 (segment (start 142.087473 81.73) (end 143.61 83.252527) (width 0.4) (layer "B.Cu") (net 3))
 (segment (start 121.265 82.894128) (end 122.429128 81.73) (width 0.4) (layer "B.Cu") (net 3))
 (segment (start 122.429128 81.73) (end 142.087473 81.73) (width 0.4) (layer "B.Cu") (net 3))
 (segment (start 121.265 84.99) (end 121.265 82.894128) (width 0.4) (layer "B.Cu") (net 3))
 (segment (start 143.61 84.99) (end 142.24 86.36) (width 0.4) (layer "B.Cu") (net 3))
 (segment (start 122.635 86.36) (end 121.265 84.99) (width 0.4) (layer "B.Cu") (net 3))
 (segment (start 139.7 91.44) (end 125.175 91.44) (width 0.4) (layer "B.Cu") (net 8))
 (segment (start 125.175 83.82) (end 139.7 83.82) (width 0.4) (layer "B.Cu") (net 2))
 (segment (start 144.33 86.81) (end 142.24 88.9) (width 0.4) (layer "B.Cu") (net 5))
 (segment (start 120.545 86.81) (end 120.545 82.595894) (width 0.4) (layer "B.Cu") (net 5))
 (segment (start 142.385707 81.01) (end 144.33 82.954293) (width 0.4) (layer "B.Cu") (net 5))
 (segment (start 122.635 88.9) (end 120.545 86.81) (width 0.4) (layer "B.Cu") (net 5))
 (segment (start 144.33 82.954293) (end 144.33 86.81) (width 0.4) (layer "B.Cu") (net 5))
 (segment (start 122.130894 81.01) (end 142.385707 81.01) (width 0.4) (layer "B.Cu") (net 5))
 (segment (start 120.545 82.595894) (end 122.130894 81.01) (width 0.4) (layer "B.Cu") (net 5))
 (segment (start 139.7 96.52) (end 125.175 96.52) (width 0.4) (layer "B.Cu") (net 12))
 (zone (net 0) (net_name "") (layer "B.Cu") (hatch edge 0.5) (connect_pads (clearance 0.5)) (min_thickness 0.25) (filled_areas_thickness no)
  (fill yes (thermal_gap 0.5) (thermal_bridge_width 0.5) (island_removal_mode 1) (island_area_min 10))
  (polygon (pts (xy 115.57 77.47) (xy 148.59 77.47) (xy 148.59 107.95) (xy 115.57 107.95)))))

